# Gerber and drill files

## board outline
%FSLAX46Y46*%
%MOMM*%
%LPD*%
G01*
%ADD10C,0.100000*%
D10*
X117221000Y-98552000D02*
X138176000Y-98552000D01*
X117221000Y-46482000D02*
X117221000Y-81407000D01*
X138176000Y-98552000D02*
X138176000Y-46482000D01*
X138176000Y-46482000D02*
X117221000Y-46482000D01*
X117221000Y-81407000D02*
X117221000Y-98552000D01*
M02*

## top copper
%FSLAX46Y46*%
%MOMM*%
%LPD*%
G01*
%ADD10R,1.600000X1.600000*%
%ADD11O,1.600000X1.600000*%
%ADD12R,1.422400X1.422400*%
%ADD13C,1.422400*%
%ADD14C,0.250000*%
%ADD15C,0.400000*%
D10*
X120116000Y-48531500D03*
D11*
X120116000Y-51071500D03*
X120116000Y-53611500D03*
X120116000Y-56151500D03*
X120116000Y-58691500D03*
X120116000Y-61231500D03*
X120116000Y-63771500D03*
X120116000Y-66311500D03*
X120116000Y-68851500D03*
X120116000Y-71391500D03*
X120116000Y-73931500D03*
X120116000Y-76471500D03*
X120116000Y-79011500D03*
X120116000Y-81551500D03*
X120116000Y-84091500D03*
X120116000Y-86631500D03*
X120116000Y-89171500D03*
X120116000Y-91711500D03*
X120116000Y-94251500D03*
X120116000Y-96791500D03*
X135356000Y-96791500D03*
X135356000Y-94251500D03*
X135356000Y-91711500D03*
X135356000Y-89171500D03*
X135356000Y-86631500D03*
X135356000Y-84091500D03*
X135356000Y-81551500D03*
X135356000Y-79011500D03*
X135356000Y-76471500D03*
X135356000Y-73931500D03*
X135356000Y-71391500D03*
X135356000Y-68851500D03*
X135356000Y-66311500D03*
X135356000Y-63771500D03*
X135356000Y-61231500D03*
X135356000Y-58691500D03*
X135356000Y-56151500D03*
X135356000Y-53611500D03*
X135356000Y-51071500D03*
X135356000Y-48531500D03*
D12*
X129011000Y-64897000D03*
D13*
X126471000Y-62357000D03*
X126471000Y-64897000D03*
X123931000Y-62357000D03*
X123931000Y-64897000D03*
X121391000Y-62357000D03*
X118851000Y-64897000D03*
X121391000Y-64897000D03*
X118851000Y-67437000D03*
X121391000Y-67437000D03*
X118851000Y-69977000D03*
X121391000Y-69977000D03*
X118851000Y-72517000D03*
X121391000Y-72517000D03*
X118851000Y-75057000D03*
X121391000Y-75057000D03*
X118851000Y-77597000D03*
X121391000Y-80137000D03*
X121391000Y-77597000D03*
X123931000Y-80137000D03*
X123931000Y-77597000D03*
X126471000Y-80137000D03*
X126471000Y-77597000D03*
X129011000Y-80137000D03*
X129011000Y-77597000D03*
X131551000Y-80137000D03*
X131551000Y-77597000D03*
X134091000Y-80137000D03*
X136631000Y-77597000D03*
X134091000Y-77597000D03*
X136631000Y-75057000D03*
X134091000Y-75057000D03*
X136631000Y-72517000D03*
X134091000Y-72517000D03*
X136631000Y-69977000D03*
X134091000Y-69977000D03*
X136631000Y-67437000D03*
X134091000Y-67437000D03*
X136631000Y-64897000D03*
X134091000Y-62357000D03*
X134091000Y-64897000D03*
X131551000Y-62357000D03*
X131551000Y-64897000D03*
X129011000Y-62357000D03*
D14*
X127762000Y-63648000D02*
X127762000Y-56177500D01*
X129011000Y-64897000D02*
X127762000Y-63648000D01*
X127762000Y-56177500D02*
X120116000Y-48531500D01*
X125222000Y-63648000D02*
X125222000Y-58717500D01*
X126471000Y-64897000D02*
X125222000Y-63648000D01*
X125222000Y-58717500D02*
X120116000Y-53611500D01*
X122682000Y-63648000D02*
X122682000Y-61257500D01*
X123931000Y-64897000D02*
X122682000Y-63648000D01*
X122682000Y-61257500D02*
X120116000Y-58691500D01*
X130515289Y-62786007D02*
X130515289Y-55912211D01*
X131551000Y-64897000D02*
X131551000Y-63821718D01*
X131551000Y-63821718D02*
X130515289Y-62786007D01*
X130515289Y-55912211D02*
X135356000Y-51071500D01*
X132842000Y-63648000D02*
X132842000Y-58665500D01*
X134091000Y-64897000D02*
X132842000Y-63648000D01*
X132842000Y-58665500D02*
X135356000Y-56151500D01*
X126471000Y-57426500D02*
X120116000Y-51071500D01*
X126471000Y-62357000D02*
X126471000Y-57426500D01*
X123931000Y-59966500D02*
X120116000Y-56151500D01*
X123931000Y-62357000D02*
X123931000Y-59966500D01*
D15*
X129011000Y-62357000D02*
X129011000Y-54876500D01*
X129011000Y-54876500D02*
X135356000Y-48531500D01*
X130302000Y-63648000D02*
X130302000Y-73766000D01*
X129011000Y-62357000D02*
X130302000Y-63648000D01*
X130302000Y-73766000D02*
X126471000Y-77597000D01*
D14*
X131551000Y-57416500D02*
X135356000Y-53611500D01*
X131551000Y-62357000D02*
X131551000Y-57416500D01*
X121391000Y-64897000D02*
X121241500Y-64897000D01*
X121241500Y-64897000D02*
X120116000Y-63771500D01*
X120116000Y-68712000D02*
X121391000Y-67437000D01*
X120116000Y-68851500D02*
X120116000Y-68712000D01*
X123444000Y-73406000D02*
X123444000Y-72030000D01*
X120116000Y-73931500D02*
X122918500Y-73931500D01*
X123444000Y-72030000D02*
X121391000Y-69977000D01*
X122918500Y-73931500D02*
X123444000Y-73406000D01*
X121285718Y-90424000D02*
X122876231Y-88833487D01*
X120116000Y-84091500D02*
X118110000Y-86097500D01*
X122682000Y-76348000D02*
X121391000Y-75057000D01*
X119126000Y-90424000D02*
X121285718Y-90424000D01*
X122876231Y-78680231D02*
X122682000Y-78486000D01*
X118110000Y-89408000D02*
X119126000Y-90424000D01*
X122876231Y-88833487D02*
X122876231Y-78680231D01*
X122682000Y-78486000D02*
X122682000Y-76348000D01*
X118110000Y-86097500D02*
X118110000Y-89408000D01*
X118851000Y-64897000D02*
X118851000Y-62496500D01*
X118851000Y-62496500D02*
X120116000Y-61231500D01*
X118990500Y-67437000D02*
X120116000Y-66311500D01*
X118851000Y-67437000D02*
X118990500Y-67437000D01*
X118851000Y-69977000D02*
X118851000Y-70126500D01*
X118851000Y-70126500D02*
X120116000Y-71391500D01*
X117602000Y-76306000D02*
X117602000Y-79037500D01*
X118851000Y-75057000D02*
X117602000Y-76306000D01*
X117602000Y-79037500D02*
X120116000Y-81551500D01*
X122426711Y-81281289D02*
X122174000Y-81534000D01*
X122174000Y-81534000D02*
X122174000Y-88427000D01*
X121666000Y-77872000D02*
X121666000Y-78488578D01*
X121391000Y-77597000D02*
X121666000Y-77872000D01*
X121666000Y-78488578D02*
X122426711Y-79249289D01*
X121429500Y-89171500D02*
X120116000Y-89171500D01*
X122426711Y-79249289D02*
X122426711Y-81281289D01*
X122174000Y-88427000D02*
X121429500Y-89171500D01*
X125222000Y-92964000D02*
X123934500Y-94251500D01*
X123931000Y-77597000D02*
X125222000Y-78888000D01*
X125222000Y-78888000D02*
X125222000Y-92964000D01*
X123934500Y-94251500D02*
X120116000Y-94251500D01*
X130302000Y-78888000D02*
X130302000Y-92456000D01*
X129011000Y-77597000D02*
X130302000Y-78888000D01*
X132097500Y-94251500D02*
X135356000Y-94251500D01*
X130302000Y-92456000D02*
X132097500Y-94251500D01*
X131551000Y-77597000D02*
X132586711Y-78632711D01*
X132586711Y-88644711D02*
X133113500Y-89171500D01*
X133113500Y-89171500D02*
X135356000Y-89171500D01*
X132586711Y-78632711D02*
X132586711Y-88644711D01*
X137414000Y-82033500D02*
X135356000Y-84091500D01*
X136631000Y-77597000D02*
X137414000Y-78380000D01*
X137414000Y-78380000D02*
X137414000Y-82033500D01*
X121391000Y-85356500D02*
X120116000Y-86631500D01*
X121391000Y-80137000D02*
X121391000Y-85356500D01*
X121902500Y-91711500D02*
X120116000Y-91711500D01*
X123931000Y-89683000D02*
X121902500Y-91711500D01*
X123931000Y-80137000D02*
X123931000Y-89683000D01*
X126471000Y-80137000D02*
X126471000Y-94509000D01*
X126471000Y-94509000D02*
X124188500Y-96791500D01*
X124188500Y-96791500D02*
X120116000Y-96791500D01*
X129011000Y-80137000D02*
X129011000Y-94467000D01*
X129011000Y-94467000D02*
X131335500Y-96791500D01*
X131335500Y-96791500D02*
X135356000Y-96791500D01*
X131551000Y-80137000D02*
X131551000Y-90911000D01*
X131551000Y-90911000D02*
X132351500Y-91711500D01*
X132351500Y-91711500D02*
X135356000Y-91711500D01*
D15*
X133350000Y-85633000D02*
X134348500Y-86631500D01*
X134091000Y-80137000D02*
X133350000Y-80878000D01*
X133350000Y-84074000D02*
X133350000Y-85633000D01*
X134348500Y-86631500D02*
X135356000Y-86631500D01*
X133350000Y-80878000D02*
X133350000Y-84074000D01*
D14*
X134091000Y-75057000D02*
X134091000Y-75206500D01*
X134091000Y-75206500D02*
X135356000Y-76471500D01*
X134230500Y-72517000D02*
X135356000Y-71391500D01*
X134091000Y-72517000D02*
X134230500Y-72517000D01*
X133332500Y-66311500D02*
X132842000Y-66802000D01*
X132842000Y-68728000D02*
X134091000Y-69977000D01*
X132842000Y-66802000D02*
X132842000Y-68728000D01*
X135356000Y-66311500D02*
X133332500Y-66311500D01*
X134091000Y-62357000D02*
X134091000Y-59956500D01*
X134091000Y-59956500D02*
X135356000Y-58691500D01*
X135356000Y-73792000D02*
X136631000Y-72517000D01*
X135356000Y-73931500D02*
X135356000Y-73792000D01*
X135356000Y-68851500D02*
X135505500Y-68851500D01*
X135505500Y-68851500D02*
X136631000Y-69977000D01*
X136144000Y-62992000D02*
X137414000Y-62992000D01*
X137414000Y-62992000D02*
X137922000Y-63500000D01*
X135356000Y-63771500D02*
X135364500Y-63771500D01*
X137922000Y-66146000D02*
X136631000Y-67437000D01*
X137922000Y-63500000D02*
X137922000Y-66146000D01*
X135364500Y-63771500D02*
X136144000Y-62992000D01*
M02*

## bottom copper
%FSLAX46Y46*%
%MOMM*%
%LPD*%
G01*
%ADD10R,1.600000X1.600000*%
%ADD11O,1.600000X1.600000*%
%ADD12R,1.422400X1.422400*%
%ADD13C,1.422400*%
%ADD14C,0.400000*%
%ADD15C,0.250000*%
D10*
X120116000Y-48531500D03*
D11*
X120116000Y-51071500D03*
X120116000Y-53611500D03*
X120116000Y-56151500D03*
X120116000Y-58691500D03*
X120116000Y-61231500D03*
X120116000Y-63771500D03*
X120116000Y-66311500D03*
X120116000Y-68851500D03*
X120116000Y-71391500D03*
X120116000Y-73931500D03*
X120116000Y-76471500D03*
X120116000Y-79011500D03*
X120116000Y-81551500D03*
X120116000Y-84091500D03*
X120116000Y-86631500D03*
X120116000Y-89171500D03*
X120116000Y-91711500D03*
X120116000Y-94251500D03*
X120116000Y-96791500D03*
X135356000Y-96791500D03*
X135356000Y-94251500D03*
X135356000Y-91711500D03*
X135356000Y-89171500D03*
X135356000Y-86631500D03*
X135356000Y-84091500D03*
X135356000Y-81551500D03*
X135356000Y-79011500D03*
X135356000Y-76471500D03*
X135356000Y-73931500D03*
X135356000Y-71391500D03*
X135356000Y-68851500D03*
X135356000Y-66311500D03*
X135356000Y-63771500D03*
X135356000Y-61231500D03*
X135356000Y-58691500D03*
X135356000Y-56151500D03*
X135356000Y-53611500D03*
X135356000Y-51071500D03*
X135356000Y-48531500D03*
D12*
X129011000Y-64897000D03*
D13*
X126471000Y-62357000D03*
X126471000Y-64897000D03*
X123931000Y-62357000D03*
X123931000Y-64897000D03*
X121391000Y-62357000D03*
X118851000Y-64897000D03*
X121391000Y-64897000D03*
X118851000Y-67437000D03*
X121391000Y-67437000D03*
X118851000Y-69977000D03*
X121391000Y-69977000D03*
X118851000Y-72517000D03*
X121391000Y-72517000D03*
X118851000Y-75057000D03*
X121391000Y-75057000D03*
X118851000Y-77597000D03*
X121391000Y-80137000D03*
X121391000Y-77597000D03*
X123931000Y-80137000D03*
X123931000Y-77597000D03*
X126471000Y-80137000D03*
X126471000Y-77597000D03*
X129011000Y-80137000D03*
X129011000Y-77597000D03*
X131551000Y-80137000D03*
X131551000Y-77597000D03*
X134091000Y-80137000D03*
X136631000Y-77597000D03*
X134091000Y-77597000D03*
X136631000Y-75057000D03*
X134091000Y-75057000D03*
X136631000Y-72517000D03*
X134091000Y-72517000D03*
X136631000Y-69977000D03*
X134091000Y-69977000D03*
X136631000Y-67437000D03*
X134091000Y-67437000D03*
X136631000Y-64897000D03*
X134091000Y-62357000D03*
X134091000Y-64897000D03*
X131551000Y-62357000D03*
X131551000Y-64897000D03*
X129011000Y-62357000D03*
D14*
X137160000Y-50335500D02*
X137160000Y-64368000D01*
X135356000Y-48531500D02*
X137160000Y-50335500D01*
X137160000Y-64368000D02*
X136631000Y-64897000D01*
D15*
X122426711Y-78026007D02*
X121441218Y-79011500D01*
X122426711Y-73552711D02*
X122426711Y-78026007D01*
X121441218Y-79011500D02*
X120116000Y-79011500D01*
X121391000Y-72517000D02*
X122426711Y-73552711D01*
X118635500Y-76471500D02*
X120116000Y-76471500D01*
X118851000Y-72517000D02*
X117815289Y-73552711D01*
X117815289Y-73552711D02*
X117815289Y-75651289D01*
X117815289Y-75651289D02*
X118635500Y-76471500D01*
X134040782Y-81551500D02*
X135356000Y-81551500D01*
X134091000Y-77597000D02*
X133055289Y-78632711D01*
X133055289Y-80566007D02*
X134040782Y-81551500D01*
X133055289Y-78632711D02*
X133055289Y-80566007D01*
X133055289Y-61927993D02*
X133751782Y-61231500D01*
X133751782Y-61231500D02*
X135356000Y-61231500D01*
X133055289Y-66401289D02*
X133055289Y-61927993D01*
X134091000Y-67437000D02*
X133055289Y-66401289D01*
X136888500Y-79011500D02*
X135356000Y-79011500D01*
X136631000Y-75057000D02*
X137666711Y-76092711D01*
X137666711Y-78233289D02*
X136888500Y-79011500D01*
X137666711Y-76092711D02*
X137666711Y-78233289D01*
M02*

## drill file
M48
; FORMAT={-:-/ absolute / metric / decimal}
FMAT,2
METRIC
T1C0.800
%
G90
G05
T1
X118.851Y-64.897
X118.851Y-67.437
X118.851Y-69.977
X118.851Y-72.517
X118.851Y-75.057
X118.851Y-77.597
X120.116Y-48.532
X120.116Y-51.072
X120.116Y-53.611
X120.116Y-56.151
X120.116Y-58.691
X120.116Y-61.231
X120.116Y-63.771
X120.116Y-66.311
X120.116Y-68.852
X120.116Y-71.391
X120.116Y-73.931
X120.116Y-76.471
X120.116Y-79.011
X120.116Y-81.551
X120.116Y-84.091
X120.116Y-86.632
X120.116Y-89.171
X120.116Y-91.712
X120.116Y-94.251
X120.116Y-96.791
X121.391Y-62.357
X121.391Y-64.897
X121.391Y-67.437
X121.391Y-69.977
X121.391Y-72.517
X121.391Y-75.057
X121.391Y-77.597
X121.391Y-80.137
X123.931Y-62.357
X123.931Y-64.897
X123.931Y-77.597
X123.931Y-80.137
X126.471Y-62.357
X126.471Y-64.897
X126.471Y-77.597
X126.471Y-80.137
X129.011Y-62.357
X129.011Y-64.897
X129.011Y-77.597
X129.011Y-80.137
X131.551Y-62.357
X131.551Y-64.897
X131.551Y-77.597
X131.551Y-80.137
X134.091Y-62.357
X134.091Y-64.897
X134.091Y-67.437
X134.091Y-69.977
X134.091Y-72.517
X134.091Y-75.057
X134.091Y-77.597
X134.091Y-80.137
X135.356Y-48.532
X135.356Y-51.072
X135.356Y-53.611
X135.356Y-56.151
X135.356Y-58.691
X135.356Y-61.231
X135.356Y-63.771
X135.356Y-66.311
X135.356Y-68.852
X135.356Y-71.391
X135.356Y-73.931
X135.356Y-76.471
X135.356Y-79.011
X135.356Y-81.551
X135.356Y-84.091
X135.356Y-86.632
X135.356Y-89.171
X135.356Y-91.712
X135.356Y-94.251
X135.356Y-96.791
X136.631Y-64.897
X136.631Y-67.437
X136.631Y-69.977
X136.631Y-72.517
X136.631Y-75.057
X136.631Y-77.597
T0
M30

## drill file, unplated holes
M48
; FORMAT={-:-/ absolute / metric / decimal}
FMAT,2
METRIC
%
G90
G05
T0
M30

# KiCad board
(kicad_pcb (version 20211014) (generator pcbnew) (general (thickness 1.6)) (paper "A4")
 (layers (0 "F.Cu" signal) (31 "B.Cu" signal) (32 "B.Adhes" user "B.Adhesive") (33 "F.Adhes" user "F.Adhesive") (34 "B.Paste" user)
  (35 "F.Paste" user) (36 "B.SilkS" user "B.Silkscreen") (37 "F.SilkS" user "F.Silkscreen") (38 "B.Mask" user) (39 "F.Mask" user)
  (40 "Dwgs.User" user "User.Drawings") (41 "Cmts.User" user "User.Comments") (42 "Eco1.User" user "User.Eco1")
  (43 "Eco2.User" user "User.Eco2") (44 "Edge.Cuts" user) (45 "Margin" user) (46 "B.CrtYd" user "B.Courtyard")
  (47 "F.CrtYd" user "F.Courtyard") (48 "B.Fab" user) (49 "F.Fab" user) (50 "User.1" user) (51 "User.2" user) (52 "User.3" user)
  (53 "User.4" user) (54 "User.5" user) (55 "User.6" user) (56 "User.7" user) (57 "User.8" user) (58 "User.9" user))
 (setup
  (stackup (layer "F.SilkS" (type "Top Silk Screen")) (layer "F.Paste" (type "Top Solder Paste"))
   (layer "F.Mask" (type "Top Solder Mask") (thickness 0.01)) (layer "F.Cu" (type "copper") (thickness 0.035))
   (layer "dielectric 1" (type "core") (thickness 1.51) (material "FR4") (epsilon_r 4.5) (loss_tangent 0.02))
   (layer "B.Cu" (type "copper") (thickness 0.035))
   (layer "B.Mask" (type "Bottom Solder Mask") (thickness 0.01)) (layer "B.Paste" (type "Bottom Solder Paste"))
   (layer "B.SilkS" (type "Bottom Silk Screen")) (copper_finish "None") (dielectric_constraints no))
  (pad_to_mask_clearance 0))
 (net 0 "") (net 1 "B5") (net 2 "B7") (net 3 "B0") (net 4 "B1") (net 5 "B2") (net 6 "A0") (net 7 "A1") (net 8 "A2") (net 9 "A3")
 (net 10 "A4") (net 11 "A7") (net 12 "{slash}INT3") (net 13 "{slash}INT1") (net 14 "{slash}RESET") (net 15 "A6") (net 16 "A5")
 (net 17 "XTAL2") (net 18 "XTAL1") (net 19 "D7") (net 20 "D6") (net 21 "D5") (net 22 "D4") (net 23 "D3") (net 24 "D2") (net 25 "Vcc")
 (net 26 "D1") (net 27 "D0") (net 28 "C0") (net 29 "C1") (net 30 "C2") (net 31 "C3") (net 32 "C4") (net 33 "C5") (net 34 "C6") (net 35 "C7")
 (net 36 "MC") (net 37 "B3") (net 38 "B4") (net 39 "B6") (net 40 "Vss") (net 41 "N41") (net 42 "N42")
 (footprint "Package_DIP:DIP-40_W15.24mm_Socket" (layer "F.Cu") (at 120.116 48.5315)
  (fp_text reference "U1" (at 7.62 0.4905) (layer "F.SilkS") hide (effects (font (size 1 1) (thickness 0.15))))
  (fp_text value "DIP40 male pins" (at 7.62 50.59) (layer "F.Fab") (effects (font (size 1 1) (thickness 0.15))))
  (pad "1" thru_hole rect locked (at 0 0) (size 1.6 1.6) (drill 0.8) (layers *.Cu *.Mask) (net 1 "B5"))
  (pad "2" thru_hole oval locked (at 0 2.54) (size 1.6 1.6) (drill 0.8) (layers *.Cu *.Mask) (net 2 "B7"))
  (pad "3" thru_hole oval locked (at 0 5.08) (size 1.6 1.6) (drill 0.8) (layers *.Cu *.Mask) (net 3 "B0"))
  (pad "4" thru_hole oval locked (at 0 7.62) (size 1.6 1.6) (drill 0.8) (layers *.Cu *.Mask) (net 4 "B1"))
  (pad "5" thru_hole oval locked (at 0 10.16) (size 1.6 1.6) (drill 0.8) (layers *.Cu *.Mask) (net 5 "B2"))
  (pad "6" thru_hole oval locked (at 0 12.7) (size 1.6 1.6) (drill 0.8) (layers *.Cu *.Mask) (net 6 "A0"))
  (pad "7" thru_hole oval locked (at 0 15.24) (size 1.6 1.6) (drill 0.8) (layers *.Cu *.Mask) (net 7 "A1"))
  (pad "8" thru_hole oval locked (at 0 17.78) (size 1.6 1.6) (drill 0.8) (layers *.Cu *.Mask) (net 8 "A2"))
  (pad "9" thru_hole oval locked (at 0 20.32) (size 1.6 1.6) (drill 0.8) (layers *.Cu *.Mask) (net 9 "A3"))
  (pad "10" thru_hole oval locked (at 0 22.86) (size 1.6 1.6) (drill 0.8) (layers *.Cu *.Mask) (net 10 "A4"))
  (pad "11" thru_hole oval locked (at 0 25.4) (size 1.6 1.6) (drill 0.8) (layers *.Cu *.Mask) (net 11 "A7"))
  (pad "12" thru_hole oval locked (at 0 27.94) (size 1.6 1.6) (drill 0.8) (layers *.Cu *.Mask) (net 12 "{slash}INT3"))
  (pad "13" thru_hole oval locked (at 0 30.48) (size 1.6 1.6) (drill 0.8) (layers *.Cu *.Mask) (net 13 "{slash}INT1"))
  (pad "14" thru_hole oval locked (at 0 33.02) (size 1.6 1.6) (drill 0.8) (layers *.Cu *.Mask) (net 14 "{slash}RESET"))
  (pad "15" thru_hole oval locked (at 0 35.56) (size 1.6 1.6) (drill 0.8) (layers *.Cu *.Mask) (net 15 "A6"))
  (pad "16" thru_hole oval locked (at 0 38.1) (size 1.6 1.6) (drill 0.8) (layers *.Cu *.Mask) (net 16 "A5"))
  (pad "17" thru_hole oval locked (at 0 40.64) (size 1.6 1.6) (drill 0.8) (layers *.Cu *.Mask) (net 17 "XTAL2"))
  (pad "18" thru_hole oval locked (at 0 43.18) (size 1.6 1.6) (drill 0.8) (layers *.Cu *.Mask) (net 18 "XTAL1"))
  (pad "19" thru_hole oval locked (at 0 45.72) (size 1.6 1.6) (drill 0.8) (layers *.Cu *.Mask) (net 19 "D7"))
  (pad "20" thru_hole oval locked (at 0 48.26) (size 1.6 1.6) (drill 0.8) (layers *.Cu *.Mask) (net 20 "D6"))
  (pad "21" thru_hole oval locked (at 15.24 48.26) (size 1.6 1.6) (drill 0.8) (layers *.Cu *.Mask) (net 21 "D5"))
  (pad "22" thru_hole oval locked (at 15.24 45.72) (size 1.6 1.6) (drill 0.8) (layers *.Cu *.Mask) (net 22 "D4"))
  (pad "23" thru_hole oval locked (at 15.24 43.18) (size 1.6 1.6) (drill 0.8) (layers *.Cu *.Mask) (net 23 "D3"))
  (pad "24" thru_hole oval locked (at 15.24 40.64) (size 1.6 1.6) (drill 0.8) (layers *.Cu *.Mask) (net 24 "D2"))
  (pad "25" thru_hole oval locked (at 15.24 38.1) (size 1.6 1.6) (drill 0.8) (layers *.Cu *.Mask) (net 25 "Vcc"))
  (pad "26" thru_hole oval locked (at 15.24 35.56) (size 1.6 1.6) (drill 0.8) (layers *.Cu *.Mask) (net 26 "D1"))
  (pad "27" thru_hole oval locked (at 15.24 33.02) (size 1.6 1.6) (drill 0.8) (layers *.Cu *.Mask) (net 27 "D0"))
  (pad "28" thru_hole oval locked (at 15.24 30.48) (size 1.6 1.6) (drill 0.8) (layers *.Cu *.Mask) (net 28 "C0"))
  (pad "29" thru_hole oval locked (at 15.24 27.94) (size 1.6 1.6) (drill 0.8) (layers *.Cu *.Mask) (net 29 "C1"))
  (pad "30" thru_hole oval locked (at 15.24 25.4) (size 1.6 1.6) (drill 0.8) (layers *.Cu *.Mask) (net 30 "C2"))
  (pad "31" thru_hole oval locked (at 15.24 22.86) (size 1.6 1.6) (drill 0.8) (layers *.Cu *.Mask) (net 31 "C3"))
  (pad "32" thru_hole oval locked (at 15.24 20.32) (size 1.6 1.6) (drill 0.8) (layers *.Cu *.Mask) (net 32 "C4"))
  (pad "33" thru_hole oval locked (at 15.24 17.78) (size 1.6 1.6) (drill 0.8) (layers *.Cu *.Mask) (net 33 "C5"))
  (pad "34" thru_hole oval locked (at 15.24 15.24) (size 1.6 1.6) (drill 0.8) (layers *.Cu *.Mask) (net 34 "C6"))
  (pad "35" thru_hole oval locked (at 15.24 12.7) (size 1.6 1.6) (drill 0.8) (layers *.Cu *.Mask) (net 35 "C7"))
  (pad "36" thru_hole oval locked (at 15.24 10.16) (size 1.6 1.6) (drill 0.8) (layers *.Cu *.Mask) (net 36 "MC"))
  (pad "37" thru_hole oval locked (at 15.24 7.62) (size 1.6 1.6) (drill 0.8) (layers *.Cu *.Mask) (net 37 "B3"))
  (pad "38" thru_hole oval locked (at 15.24 5.08) (size 1.6 1.6) (drill 0.8) (layers *.Cu *.Mask) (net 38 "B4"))
  (pad "39" thru_hole oval locked (at 15.24 2.54) (size 1.6 1.6) (drill 0.8) (layers *.Cu *.Mask) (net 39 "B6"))
  (pad "40" thru_hole oval locked (at 15.24 0) (size 1.6 1.6) (drill 0.8) (layers *.Cu *.Mask) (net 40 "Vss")))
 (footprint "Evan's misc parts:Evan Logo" (layer "F.Cu") (at 127.381 91.567)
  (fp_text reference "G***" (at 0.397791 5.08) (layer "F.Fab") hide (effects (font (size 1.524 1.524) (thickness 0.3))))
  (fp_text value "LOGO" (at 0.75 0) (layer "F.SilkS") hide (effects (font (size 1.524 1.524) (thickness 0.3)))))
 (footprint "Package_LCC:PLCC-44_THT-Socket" (layer "F.Cu") (at 129.011 64.897)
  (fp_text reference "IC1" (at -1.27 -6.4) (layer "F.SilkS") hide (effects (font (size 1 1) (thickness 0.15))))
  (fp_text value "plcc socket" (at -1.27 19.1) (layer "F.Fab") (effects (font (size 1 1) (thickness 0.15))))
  (pad "1" thru_hole rect locked (at 0 0) (size 1.4224 1.4224) (drill 0.8) (layers *.Cu *.Mask) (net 1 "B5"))
  (pad "2" thru_hole circle locked (at -2.54 -2.54) (size 1.4224 1.4224) (drill 0.8) (layers *.Cu *.Mask) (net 2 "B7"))
  (pad "3" thru_hole circle locked (at -2.54 0) (size 1.4224 1.4224) (drill 0.8) (layers *.Cu *.Mask) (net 3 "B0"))
  (pad "4" thru_hole circle locked (at -5.08 -2.54) (size 1.4224 1.4224) (drill 0.8) (layers *.Cu *.Mask) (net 4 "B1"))
  (pad "5" thru_hole circle locked (at -5.08 0) (size 1.4224 1.4224) (drill 0.8) (layers *.Cu *.Mask) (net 5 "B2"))
  (pad "6" thru_hole circle locked (at -7.62 -2.54) (size 1.4224 1.4224) (drill 0.8) (layers *.Cu *.Mask) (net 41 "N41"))
  (pad "7" thru_hole circle locked (at -10.16 0) (size 1.4224 1.4224) (drill 0.8) (layers *.Cu *.Mask) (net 6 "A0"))
  (pad "8" thru_hole circle locked (at -7.62 0) (size 1.4224 1.4224) (drill 0.8) (layers *.Cu *.Mask) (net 7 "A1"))
  (pad "9" thru_hole circle locked (at -10.16 2.54) (size 1.4224 1.4224) (drill 0.8) (layers *.Cu *.Mask) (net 8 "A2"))
  (pad "10" thru_hole circle locked (at -7.62 2.54) (size 1.4224 1.4224) (drill 0.8) (layers *.Cu *.Mask) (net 9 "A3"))
  (pad "11" thru_hole circle locked (at -10.16 5.08) (size 1.4224 1.4224) (drill 0.8) (layers *.Cu *.Mask) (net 10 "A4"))
  (pad "12" thru_hole circle locked (at -7.62 5.08) (size 1.4224 1.4224) (drill 0.8) (layers *.Cu *.Mask) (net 11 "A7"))
  (pad "13" thru_hole circle locked (at -10.16 7.62) (size 1.4224 1.4224) (drill 0.8) (layers *.Cu *.Mask) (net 12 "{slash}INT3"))
  (pad "14" thru_hole circle locked (at -7.62 7.62) (size 1.4224 1.4224) (drill 0.8) (layers *.Cu *.Mask) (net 13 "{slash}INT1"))
  (pad "15" thru_hole circle locked (at -10.16 10.16) (size 1.4224 1.4224) (drill 0.8) (layers *.Cu *.Mask) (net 14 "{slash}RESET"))
  (pad "16" thru_hole circle locked (at -7.62 10.16) (size 1.4224 1.4224) (drill 0.8) (layers *.Cu *.Mask) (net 15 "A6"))
  (pad "17" thru_hole circle locked (at -10.16 12.7) (size 1.4224 1.4224) (drill 0.8) (layers *.Cu *.Mask) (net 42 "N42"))
  (pad "18" thru_hole circle locked (at -7.62 15.24) (size 1.4224 1.4224) (drill 0.8) (layers *.Cu *.Mask) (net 16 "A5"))
  (pad "19" thru_hole circle locked (at -7.62 12.7) (size 1.4224 1.4224) (drill 0.8) (layers *.Cu *.Mask) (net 17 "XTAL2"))
  (pad "20" thru_hole circle locked (at -5.08 15.24) (size 1.4224 1.4224) (drill 0.8) (layers *.Cu *.Mask) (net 18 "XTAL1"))
  (pad "21" thru_hole circle locked (at -5.08 12.7) (size 1.4224 1.4224) (drill 0.8) (layers *.Cu *.Mask) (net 19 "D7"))
  (pad "22" thru_hole circle locked (at -2.54 15.24) (size 1.4224 1.4224) (drill 0.8) (layers *.Cu *.Mask) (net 20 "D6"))
  (pad "23" thru_hole circle locked (at -2.54 12.7) (size 1.4224 1.4224) (drill 0.8) (layers *.Cu *.Mask) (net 40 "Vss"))
  (pad "24" thru_hole circle locked (at 0 15.24) (size 1.4224 1.4224) (drill 0.8) (layers *.Cu *.Mask) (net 21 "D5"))
  (pad "25" thru_hole circle locked (at 0 12.7) (size 1.4224 1.4224) (drill 0.8) (layers *.Cu *.Mask) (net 22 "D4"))
  (pad "26" thru_hole circle locked (at 2.54 15.24) (size 1.4224 1.4224) (drill 0.8) (layers *.Cu *.Mask) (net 23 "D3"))
  (pad "27" thru_hole circle locked (at 2.54 12.7) (size 1.4224 1.4224) (drill 0.8) (layers *.Cu *.Mask) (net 24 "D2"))
  (pad "28" thru_hole circle locked (at 5.08 15.24) (size 1.4224 1.4224) (drill 0.8) (layers *.Cu *.Mask) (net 25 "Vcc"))
  (pad "29" thru_hole circle locked (at 7.62 12.7) (size 1.4224 1.4224) (drill 0.8) (layers *.Cu *.Mask) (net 26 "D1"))
  (pad "30" thru_hole circle locked (at 5.08 12.7) (size 1.4224 1.4224) (drill 0.8) (layers *.Cu *.Mask) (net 27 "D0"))
  (pad "31" thru_hole circle locked (at 7.62 10.16) (size 1.4224 1.4224) (drill 0.8) (layers *.Cu *.Mask) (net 28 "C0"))
  (pad "32" thru_hole circle locked (at 5.08 10.16) (size 1.4224 1.4224) (drill 0.8) (layers *.Cu *.Mask) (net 29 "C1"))
  (pad "33" thru_hole circle locked (at 7.62 7.62) (size 1.4224 1.4224) (drill 0.8) (layers *.Cu *.Mask) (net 30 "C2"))
  (pad "34" thru_hole circle locked (at 5.08 7.62) (size 1.4224 1.4224) (drill 0.8) (layers *.Cu *.Mask) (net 31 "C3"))
  (pad "35" thru_hole circle locked (at 7.62 5.08) (size 1.4224 1.4224) (drill 0.8) (layers *.Cu *.Mask) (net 32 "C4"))
  (pad "36" thru_hole circle locked (at 5.08 5.08) (size 1.4224 1.4224) (drill 0.8) (layers *.Cu *.Mask) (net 33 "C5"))
  (pad "37" thru_hole circle locked (at 7.62 2.54) (size 1.4224 1.4224) (drill 0.8) (layers *.Cu *.Mask) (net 34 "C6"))
  (pad "38" thru_hole circle locked (at 5.08 2.54) (size 1.4224 1.4224) (drill 0.8) (layers *.Cu *.Mask) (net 35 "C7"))
  (pad "39" thru_hole circle locked (at 7.62 0) (size 1.4224 1.4224) (drill 0.8) (layers *.Cu *.Mask) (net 40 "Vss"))
  (pad "40" thru_hole circle locked (at 5.08 -2.54) (size 1.4224 1.4224) (drill 0.8) (layers *.Cu *.Mask) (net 36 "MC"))
  (pad "41" thru_hole circle locked (at 5.08 0) (size 1.4224 1.4224) (drill 0.8) (layers *.Cu *.Mask) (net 37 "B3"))
  (pad "42" thru_hole circle locked (at 2.54 -2.54) (size 1.4224 1.4224) (drill 0.8) (layers *.Cu *.Mask) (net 38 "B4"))
  (pad "43" thru_hole circle locked (at 2.54 0) (size 1.4224 1.4224) (drill 0.8) (layers *.Cu *.Mask) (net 39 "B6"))
  (pad "44" thru_hole circle locked (at 0 -2.54) (size 1.4224 1.4224) (drill 0.8) (layers *.Cu *.Mask) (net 40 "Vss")))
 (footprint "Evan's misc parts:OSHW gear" (layer "B.Cu") (at 127.381 90.932 180)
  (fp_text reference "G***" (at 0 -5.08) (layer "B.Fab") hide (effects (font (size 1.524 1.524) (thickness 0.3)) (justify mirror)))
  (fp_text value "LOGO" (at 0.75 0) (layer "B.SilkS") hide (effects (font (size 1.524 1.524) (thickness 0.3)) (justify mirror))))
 (gr_line (start 117.221 98.552) (end 138.176 98.552) (layer "Edge.Cuts") (width 0.1))
 (gr_line (start 117.221 46.482) (end 117.221 81.407) (layer "Edge.Cuts") (width 0.1))
 (gr_line (start 138.176 98.552) (end 138.176 46.482) (layer "Edge.Cuts") (width 0.1))
 (gr_line (start 138.176 46.482) (end 117.221 46.482) (layer "Edge.Cuts") (width 0.1))
 (gr_line (start 117.221 81.407) (end 117.221 98.552) (layer "Edge.Cuts") (width 0.1))
 (segment (start 127.762 63.648) (end 127.762 56.1775) (width 0.25) (layer "F.Cu") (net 1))
 (segment (start 129.011 64.897) (end 127.762 63.648) (width 0.25) (layer "F.Cu") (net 1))
 (segment (start 127.762 56.1775) (end 120.116 48.5315) (width 0.25) (layer "F.Cu") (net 1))
 (segment (start 125.222 63.648) (end 125.222 58.7175) (width 0.25) (layer "F.Cu") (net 3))
 (segment (start 126.471 64.897) (end 125.222 63.648) (width 0.25) (layer "F.Cu") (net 3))
 (segment (start 125.222 58.7175) (end 120.116 53.6115) (width 0.25) (layer "F.Cu") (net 3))
 (segment (start 122.682 63.648) (end 122.682 61.2575) (width 0.25) (layer "F.Cu") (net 5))
 (segment (start 123.931 64.897) (end 122.682 63.648) (width 0.25) (layer "F.Cu") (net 5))
 (segment (start 122.682 61.2575) (end 120.116 58.6915) (width 0.25) (layer "F.Cu") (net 5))
 (segment (start 130.515289 62.786007) (end 130.515289 55.912211) (width 0.25) (layer "F.Cu") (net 39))
 (segment (start 131.551 64.897) (end 131.551 63.821718) (width 0.25) (layer "F.Cu") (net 39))
 (segment (start 131.551 63.821718) (end 130.515289 62.786007) (width 0.25) (layer "F.Cu") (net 39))
 (segment (start 130.515289 55.912211) (end 135.356 51.0715) (width 0.25) (layer "F.Cu") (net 39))
 (segment (start 132.842 63.648) (end 132.842 58.6655) (width 0.25) (layer "F.Cu") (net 37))
 (segment (start 134.091 64.897) (end 132.842 63.648) (width 0.25) (layer "F.Cu") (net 37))
 (segment (start 132.842 58.6655) (end 135.356 56.1515) (width 0.25) (layer "F.Cu") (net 37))
 (segment (start 126.471 57.4265) (end 120.116 51.0715) (width 0.25) (layer "F.Cu") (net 2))
 (segment (start 126.471 62.357) (end 126.471 57.4265) (width 0.25) (layer "F.Cu") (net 2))
 (segment (start 123.931 59.9665) (end 120.116 56.1515) (width 0.25) (layer "F.Cu") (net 4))
 (segment (start 123.931 62.357) (end 123.931 59.9665) (width 0.25) (layer "F.Cu") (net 4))
 (segment (start 129.011 62.357) (end 129.011 54.8765) (width 0.4) (layer "F.Cu") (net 40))
 (segment (start 129.011 54.8765) (end 135.356 48.5315) (width 0.4) (layer "F.Cu") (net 40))
 (segment (start 130.302 63.648) (end 130.302 73.766) (width 0.4) (layer "F.Cu") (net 40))
 (segment (start 129.011 62.357) (end 130.302 63.648) (width 0.4) (layer "F.Cu") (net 40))
 (segment (start 130.302 73.766) (end 126.471 77.597) (width 0.4) (layer "F.Cu") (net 40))
 (segment (start 137.16 50.3355) (end 137.16 64.368) (width 0.4) (layer "B.Cu") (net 40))
 (segment (start 135.356 48.5315) (end 137.16 50.3355) (width 0.4) (layer "B.Cu") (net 40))
 (segment (start 137.16 64.368) (end 136.631 64.897) (width 0.4) (layer "B.Cu") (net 40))
 (segment (start 131.551 57.4165) (end 135.356 53.6115) (width 0.25) (layer "F.Cu") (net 38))
 (segment (start 131.551 62.357) (end 131.551 57.4165) (width 0.25) (layer "F.Cu") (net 38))
 (segment (start 121.391 64.897) (end 121.2415 64.897) (width 0.25) (layer "F.Cu") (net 7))
 (segment (start 121.2415 64.897) (end 120.116 63.7715) (width 0.25) (layer "F.Cu") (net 7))
 (segment (start 120.116 68.712) (end 121.391 67.437) (width 0.25) (layer "F.Cu") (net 9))
 (segment (start 120.116 68.8515) (end 120.116 68.712) (width 0.25) (layer "F.Cu") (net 9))
 (segment (start 123.444 73.406) (end 123.444 72.03) (width 0.25) (layer "F.Cu") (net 11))
 (segment (start 120.116 73.9315) (end 122.9185 73.9315) (width 0.25) (layer "F.Cu") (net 11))
 (segment (start 123.444 72.03) (end 121.391 69.977) (width 0.25) (layer "F.Cu") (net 11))
 (segment (start 122.9185 73.9315) (end 123.444 73.406) (width 0.25) (layer "F.Cu") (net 11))
 (segment (start 122.426711 78.026007) (end 121.441218 79.0115) (width 0.25) (layer "B.Cu") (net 13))
 (segment (start 122.426711 73.552711) (end 122.426711 78.026007) (width 0.25) (layer "B.Cu") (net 13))
 (segment (start 121.441218 79.0115) (end 120.116 79.0115) (width 0.25) (layer "B.Cu") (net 13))
 (segment (start 121.391 72.517) (end 122.426711 73.552711) (width 0.25) (layer "B.Cu") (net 13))
 (segment (start 121.285718 90.424) (end 122.876231 88.833487) (width 0.25) (layer "F.Cu") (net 15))
 (segment (start 120.116 84.0915) (end 118.11 86.0975) (width 0.25) (layer "F.Cu") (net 15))
 (segment (start 122.682 76.348) (end 121.391 75.057) (width 0.25) (layer "F.Cu") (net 15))
 (segment (start 119.126 90.424) (end 121.285718 90.424) (width 0.25) (layer "F.Cu") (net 15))
 (segment (start 122.876231 78.680231) (end 122.682 78.486) (width 0.25) (layer "F.Cu") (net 15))
 (segment (start 118.11 89.408) (end 119.126 90.424) (width 0.25) (layer "F.Cu") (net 15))
 (segment (start 122.876231 88.833487) (end 122.876231 78.680231) (width 0.25) (layer "F.Cu") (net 15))
 (segment (start 122.682 78.486) (end 122.682 76.348) (width 0.25) (layer "F.Cu") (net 15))
 (segment (start 118.11 86.0975) (end 118.11 89.408) (width 0.25) (layer "F.Cu") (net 15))
 (segment (start 118.851 64.897) (end 118.851 62.4965) (width 0.25) (layer "F.Cu") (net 6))
 (segment (start 118.851 62.4965) (end 120.116 61.2315) (width 0.25) (layer "F.Cu") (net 6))
 (segment (start 118.9905 67.437) (end 120.116 66.3115) (width 0.25) (layer "F.Cu") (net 8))
 (segment (start 118.851 67.437) (end 118.9905 67.437) (width 0.25) (layer "F.Cu") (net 8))
 (segment (start 118.851 69.977) (end 118.851 70.1265) (width 0.25) (layer "F.Cu") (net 10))
 (segment (start 118.851 70.1265) (end 120.116 71.3915) (width 0.25) (layer "F.Cu") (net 10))
 (segment (start 118.6355 76.4715) (end 120.116 76.4715) (width 0.25) (layer "B.Cu") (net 12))
 (segment (start 118.851 72.517) (end 117.815289 73.552711) (width 0.25) (layer "B.Cu") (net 12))
 (segment (start 117.815289 73.552711) (end 117.815289 75.651289) (width 0.25) (layer "B.Cu") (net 12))
 (segment (start 117.815289 75.651289) (end 118.6355 76.4715) (width 0.25) (layer "B.Cu") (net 12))
 (segment (start 117.602 76.306) (end 117.602 79.0375) (width 0.25) (layer "F.Cu") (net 14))
 (segment (start 118.851 75.057) (end 117.602 76.306) (width 0.25) (layer "F.Cu") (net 14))
 (segment (start 117.602 79.0375) (end 120.116 81.5515) (width 0.25) (layer "F.Cu") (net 14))
 (segment (start 122.426711 81.281289) (end 122.174 81.534) (width 0.25) (layer "F.Cu") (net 17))
 (segment (start 122.174 81.534) (end 122.174 88.427) (width 0.25) (layer "F.Cu") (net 17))
 (segment (start 121.666 77.872) (end 121.666 78.488578) (width 0.25) (layer "F.Cu") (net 17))
 (segment (start 121.391 77.597) (end 121.666 77.872) (width 0.25) (layer "F.Cu") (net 17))
 (segment (start 121.666 78.488578) (end 122.426711 79.249289) (width 0.25) (layer "F.Cu") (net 17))
 (segment (start 121.4295 89.1715) (end 120.116 89.1715) (width 0.25) (layer "F.Cu") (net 17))
 (segment (start 122.426711 79.249289) (end 122.426711 81.281289) (width 0.25) (layer "F.Cu") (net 17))
 (segment (start 122.174 88.427) (end 121.4295 89.1715) (width 0.25) (layer "F.Cu") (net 17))
 (segment (start 125.222 92.964) (end 123.9345 94.2515) (width 0.25) (layer "F.Cu") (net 19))
 (segment (start 123.931 77.597) (end 125.222 78.888) (width 0.25) (layer "F.Cu") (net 19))
 (segment (start 125.222 78.888) (end 125.222 92.964) (width 0.25) (layer "F.Cu") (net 19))
 (segment (start 123.9345 94.2515) (end 120.116 94.2515) (width 0.25) (layer "F.Cu") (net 19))
 (segment (start 130.302 78.888) (end 130.302 92.456) (width 0.25) (layer "F.Cu") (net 22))
 (segment (start 129.011 77.597) (end 130.302 78.888) (width 0.25) (layer "F.Cu") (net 22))
 (segment (start 132.0975 94.2515) (end 135.356 94.2515) (width 0.25) (layer "F.Cu") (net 22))
 (segment (start 130.302 92.456) (end 132.0975 94.2515) (width 0.25) (layer "F.Cu") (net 22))
 (segment (start 131.551 77.597) (end 132.586711 78.632711) (width 0.25) (layer "F.Cu") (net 24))
 (segment (start 132.586711 88.644711) (end 133.1135 89.1715) (width 0.25) (layer "F.Cu") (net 24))
 (segment (start 133.1135 89.1715) (end 135.356 89.1715) (width 0.25) (layer "F.Cu") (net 24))
 (segment (start 132.586711 78.632711) (end 132.586711 88.644711) (width 0.25) (layer "F.Cu") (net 24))
 (segment (start 137.414 82.0335) (end 135.356 84.0915) (width 0.25) (layer "F.Cu") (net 26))
 (segment (start 136.631 77.597) (end 137.414 78.38) (width 0.25) (layer "F.Cu") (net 26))
 (segment (start 137.414 78.38) (end 137.414 82.0335) (width 0.25) (layer "F.Cu") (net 26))
 (segment (start 121.391 85.3565) (end 120.116 86.6315) (width 0.25) (layer "F.Cu") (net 16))
 (segment (start 121.391 80.137) (end 121.391 85.3565) (width 0.25) (layer "F.Cu") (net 16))
 (segment (start 121.9025 91.7115) (end 120.116 91.7115) (width 0.25) (layer "F.Cu") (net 18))
 (segment (start 123.931 89.683) (end 121.9025 91.7115) (width 0.25) (layer "F.Cu") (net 18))
 (segment (start 123.931 80.137) (end 123.931 89.683) (width 0.25) (layer "F.Cu") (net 18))
 (segment (start 126.471 80.137) (end 126.471 94.509) (width 0.25) (layer "F.Cu") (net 20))
 (segment (start 126.471 94.509) (end 124.1885 96.7915) (width 0.25) (layer "F.Cu") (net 20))
 (segment (start 124.1885 96.7915) (end 120.116 96.7915) (width 0.25) (layer "F.Cu") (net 20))
 (segment (start 129.011 80.137) (end 129.011 94.467) (width 0.25) (layer "F.Cu") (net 21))
 (segment (start 129.011 94.467) (end 131.3355 96.7915) (width 0.25) (layer "F.Cu") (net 21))
 (segment (start 131.3355 96.7915) (end 135.356 96.7915) (width 0.25) (layer "F.Cu") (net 21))
 (segment (start 131.551 80.137) (end 131.551 90.911) (width 0.25) (layer "F.Cu") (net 23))
 (segment (start 131.551 90.911) (end 132.3515 91.7115) (width 0.25) (layer "F.Cu") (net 23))
 (segment (start 132.3515 91.7115) (end 135.356 91.7115) (width 0.25) (layer "F.Cu") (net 23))
 (segment (start 133.35 85.633) (end 134.3485 86.6315) (width 0.4) (layer "F.Cu") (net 25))
 (segment (start 134.091 80.137) (end 133.35 80.878) (width 0.4) (layer "F.Cu") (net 25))
 (segment (start 133.35 84.074) (end 133.35 85.633) (width 0.4) (layer "F.Cu") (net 25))
 (segment (start 134.3485 86.6315) (end 135.356 86.6315) (width 0.4) (layer "F.Cu") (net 25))
 (segment (start 133.35 80.878) (end 133.35 84.074) (width 0.4) (layer "F.Cu") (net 25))
 (segment (start 134.040782 81.5515) (end 135.356 81.5515) (width 0.25) (layer "B.Cu") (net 27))
 (segment (start 134.091 77.597) (end 133.055289 78.632711) (width 0.25) (layer "B.Cu") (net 27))
 (segment (start 133.055289 80.566007) (end 134.040782 81.5515) (width 0.25) (layer "B.Cu") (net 27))
 (segment (start 133.055289 78.632711) (end 133.055289 80.566007) (width 0.25) (layer "B.Cu") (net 27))
 (segment (start 134.091 75.057) (end 134.091 75.2065) (width 0.25) (layer "F.Cu") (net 29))
 (segment (start 134.091 75.2065) (end 135.356 76.4715) (width 0.25) (layer "F.Cu") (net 29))
 (segment (start 134.2305 72.517) (end 135.356 71.3915) (width 0.25) (layer "F.Cu") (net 31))
 (segment (start 134.091 72.517) (end 134.2305 72.517) (width 0.25) (layer "F.Cu") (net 31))
 (segment (start 133.3325 66.3115) (end 132.842 66.802) (width 0.25) (layer "F.Cu") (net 33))
 (segment (start 132.842 68.728) (end 134.091 69.977) (width 0.25) (layer "F.Cu") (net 33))
 (segment (start 132.842 66.802) (end 132.842 68.728) (width 0.25) (layer "F.Cu") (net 33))
 (segment (start 135.356 66.3115) (end 133.3325 66.3115) (width 0.25) (layer "F.Cu") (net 33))
 (segment (start 133.055289 61.927993) (end 133.751782 61.2315) (width 0.25) (layer "B.Cu") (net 35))
 (segment (start 133.751782 61.2315) (end 135.356 61.2315) (width 0.25) (layer "B.Cu") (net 35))
 (segment (start 133.055289 66.401289) (end 133.055289 61.927993) (width 0.25) (layer "B.Cu") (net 35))
 (segment (start 134.091 67.437) (end 133.055289 66.401289) (width 0.25) (layer "B.Cu") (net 35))
 (segment (start 134.091 62.357) (end 134.091 59.9565) (width 0.25) (layer "F.Cu") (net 36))
 (segment (start 134.091 59.9565) (end 135.356 58.6915) (width 0.25) (layer "F.Cu") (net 36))
 (segment (start 136.8885 79.0115) (end 135.356 79.0115) (width 0.25) (layer "B.Cu") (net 28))
 (segment (start 136.631 75.057) (end 137.666711 76.092711) (width 0.25) (layer "B.Cu") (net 28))
 (segment (start 137.666711 78.233289) (end 136.8885 79.0115) (width 0.25) (layer "B.Cu") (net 28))
 (segment (start 137.666711 76.092711) (end 137.666711 78.233289) (width 0.25) (layer "B.Cu") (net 28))
 (segment (start 135.356 73.792) (end 136.631 72.517) (width 0.25) (layer "F.Cu") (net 30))
 (segment (start 135.356 73.9315) (end 135.356 73.792) (width 0.25) (layer "F.Cu") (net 30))
 (segment (start 135.356 68.8515) (end 135.5055 68.8515) (width 0.25) (layer "F.Cu") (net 32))
 (segment (start 135.5055 68.8515) (end 136.631 69.977) (width 0.25) (layer "F.Cu") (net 32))
 (segment (start 136.144 62.992) (end 137.414 62.992) (width 0.25) (layer "F.Cu") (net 34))
 (segment (start 137.414 62.992) (end 137.922 63.5) (width 0.25) (layer "F.Cu") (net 34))
 (segment (start 135.356 63.7715) (end 135.3645 63.7715) (width 0.25) (layer "F.Cu") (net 34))
 (segment (start 137.922 66.146) (end 136.631 67.437) (width 0.25) (layer "F.Cu") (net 34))
 (segment (start 137.922 63.5) (end 137.922 66.146) (width 0.25) (layer "F.Cu") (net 34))
 (segment (start 135.3645 63.7715) (end 136.144 62.992) (width 0.25) (layer "F.Cu") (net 34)))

